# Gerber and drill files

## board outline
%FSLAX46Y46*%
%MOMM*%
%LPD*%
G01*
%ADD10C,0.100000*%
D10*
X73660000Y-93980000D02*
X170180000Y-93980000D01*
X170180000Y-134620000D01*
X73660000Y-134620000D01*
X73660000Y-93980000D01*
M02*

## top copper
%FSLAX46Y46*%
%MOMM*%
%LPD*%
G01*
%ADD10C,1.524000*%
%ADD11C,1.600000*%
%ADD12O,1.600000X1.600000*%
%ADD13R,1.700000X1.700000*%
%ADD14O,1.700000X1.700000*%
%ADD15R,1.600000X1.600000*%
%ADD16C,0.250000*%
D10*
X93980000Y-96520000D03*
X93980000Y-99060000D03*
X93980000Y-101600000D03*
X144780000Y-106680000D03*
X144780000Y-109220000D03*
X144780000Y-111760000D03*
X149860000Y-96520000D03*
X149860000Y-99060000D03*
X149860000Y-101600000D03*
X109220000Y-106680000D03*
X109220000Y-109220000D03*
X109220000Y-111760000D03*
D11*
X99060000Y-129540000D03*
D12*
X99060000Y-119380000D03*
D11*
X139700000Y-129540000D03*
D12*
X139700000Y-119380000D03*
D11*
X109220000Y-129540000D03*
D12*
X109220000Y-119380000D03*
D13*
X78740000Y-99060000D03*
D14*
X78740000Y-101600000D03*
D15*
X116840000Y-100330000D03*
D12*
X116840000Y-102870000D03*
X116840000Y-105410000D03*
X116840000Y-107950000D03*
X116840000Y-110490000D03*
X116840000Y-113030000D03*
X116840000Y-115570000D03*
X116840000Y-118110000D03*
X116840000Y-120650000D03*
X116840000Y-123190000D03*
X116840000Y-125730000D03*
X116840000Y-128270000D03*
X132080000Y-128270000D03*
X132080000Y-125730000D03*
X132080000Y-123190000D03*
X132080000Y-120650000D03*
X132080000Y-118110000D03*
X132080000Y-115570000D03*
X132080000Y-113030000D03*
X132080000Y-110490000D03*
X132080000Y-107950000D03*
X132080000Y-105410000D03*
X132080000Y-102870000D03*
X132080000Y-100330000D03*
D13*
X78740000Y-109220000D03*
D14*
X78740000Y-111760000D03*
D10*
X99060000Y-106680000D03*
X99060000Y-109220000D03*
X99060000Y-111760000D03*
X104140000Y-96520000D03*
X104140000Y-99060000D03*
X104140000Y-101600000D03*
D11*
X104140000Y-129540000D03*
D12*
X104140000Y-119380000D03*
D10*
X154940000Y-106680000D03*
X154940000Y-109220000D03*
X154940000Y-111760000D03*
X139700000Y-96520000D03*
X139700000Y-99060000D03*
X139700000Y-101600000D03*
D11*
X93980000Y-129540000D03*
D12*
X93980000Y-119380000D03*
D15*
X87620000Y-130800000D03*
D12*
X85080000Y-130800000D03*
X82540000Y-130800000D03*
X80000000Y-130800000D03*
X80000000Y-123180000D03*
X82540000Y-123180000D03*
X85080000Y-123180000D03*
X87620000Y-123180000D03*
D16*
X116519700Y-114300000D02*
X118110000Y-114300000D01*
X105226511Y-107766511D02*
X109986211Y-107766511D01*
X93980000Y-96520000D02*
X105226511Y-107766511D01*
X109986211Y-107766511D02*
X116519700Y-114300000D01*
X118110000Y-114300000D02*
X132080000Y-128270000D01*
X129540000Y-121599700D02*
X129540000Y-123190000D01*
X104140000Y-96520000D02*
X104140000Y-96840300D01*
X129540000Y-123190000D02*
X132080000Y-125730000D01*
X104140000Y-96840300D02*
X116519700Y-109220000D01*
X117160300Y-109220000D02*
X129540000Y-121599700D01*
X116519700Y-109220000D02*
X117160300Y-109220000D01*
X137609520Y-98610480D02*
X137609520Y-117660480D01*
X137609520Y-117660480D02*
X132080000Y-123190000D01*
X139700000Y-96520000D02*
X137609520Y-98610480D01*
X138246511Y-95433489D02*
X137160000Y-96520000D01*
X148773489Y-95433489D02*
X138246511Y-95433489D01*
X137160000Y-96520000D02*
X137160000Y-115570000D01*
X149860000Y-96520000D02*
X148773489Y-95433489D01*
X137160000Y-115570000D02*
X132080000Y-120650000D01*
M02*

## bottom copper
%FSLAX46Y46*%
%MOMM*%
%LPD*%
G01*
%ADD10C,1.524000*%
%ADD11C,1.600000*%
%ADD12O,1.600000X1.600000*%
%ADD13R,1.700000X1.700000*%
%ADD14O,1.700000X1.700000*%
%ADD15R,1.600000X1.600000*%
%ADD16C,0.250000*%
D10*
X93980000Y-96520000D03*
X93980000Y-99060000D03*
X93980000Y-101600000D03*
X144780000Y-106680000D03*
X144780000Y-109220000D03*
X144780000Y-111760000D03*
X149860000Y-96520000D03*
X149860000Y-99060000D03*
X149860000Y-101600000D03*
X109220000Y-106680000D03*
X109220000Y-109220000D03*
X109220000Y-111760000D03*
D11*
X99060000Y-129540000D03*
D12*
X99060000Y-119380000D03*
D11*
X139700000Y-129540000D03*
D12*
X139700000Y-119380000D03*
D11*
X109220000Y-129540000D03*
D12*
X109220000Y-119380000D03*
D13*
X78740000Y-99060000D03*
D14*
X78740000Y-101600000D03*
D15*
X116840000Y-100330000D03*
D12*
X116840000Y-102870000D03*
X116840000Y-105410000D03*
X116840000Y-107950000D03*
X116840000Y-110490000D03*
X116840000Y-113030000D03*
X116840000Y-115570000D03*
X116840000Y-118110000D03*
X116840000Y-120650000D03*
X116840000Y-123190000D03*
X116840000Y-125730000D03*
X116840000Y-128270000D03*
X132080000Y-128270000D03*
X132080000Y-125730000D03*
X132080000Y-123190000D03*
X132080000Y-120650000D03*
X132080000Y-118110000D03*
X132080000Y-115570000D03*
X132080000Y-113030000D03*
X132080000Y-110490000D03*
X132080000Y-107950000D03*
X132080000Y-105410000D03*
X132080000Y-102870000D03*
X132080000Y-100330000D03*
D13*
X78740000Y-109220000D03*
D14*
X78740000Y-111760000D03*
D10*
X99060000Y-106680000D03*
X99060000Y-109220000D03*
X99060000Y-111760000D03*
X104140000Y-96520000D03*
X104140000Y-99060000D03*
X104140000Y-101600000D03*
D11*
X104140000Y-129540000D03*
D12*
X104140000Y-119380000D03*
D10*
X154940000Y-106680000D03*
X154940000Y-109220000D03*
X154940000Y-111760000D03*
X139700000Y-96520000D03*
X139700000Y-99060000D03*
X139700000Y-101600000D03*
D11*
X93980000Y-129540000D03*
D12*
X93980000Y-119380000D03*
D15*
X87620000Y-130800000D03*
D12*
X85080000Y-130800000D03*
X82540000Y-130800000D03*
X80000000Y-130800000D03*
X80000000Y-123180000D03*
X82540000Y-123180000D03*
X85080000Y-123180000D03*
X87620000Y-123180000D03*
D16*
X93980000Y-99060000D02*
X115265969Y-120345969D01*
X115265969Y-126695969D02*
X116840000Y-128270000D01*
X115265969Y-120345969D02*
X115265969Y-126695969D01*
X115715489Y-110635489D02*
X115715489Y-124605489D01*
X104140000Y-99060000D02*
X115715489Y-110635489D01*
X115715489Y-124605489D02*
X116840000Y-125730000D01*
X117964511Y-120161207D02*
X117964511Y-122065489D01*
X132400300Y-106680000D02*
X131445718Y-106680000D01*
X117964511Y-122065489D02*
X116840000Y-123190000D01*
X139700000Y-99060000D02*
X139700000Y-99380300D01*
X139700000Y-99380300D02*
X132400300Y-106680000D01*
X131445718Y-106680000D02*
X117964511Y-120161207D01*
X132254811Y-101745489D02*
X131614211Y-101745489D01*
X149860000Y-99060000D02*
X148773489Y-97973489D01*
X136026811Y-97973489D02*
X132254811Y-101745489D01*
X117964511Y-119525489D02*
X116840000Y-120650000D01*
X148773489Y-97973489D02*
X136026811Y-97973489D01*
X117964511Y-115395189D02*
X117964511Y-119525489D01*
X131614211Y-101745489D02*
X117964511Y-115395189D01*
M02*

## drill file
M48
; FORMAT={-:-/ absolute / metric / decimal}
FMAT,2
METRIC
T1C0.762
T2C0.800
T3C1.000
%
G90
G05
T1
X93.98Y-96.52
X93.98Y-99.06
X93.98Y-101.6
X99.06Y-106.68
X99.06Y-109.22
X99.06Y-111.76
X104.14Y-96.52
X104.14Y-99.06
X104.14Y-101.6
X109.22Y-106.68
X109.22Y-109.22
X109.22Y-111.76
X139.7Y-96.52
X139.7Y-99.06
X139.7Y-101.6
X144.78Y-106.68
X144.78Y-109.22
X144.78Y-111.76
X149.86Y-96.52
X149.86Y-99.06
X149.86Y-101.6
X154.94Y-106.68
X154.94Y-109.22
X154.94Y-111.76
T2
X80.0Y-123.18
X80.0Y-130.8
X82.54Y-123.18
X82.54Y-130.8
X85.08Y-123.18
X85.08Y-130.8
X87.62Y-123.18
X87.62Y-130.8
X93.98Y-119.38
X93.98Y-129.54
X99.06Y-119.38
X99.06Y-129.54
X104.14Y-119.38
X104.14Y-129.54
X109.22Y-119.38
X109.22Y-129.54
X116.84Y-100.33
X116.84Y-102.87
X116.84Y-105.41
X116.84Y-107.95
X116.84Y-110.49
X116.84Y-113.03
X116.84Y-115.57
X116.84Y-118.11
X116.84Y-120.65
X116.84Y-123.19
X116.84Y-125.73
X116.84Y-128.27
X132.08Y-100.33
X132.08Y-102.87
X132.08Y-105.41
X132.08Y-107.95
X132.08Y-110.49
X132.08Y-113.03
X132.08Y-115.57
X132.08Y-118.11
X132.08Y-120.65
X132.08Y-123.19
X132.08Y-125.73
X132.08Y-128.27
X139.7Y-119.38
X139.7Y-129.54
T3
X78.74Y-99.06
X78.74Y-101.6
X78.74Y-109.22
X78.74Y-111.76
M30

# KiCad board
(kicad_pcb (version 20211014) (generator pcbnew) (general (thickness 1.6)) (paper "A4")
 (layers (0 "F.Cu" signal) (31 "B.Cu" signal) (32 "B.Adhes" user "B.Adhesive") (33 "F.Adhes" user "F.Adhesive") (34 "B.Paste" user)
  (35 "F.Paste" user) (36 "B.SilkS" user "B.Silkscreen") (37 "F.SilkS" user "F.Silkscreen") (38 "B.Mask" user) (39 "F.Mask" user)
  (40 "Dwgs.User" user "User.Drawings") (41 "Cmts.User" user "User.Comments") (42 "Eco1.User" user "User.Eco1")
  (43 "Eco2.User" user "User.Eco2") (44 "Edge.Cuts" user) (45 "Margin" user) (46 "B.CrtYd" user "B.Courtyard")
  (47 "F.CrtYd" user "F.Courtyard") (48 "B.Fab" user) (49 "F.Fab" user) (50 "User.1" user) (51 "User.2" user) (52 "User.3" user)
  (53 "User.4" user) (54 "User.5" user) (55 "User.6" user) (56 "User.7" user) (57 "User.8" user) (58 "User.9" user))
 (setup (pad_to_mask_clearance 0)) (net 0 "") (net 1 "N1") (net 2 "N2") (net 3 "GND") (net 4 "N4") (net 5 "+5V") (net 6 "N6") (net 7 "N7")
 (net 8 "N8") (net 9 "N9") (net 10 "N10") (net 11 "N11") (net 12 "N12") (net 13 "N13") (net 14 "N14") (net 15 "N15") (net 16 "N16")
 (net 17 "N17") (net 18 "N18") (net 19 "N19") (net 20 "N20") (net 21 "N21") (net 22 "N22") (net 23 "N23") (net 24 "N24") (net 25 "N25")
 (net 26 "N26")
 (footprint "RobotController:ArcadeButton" (layer "F.Cu") (at 93.98 96.52)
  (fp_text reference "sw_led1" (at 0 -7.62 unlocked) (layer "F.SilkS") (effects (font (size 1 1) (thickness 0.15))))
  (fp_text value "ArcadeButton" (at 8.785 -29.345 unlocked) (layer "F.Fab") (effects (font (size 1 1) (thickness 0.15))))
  (pad "1" thru_hole circle (at 0 0) (size 1.524 1.524) (drill 0.762) (layers *.Cu *.Mask) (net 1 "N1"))
  (pad "2" thru_hole circle (at 0 2.54) (size 1.524 1.524) (drill 0.762) (layers *.Cu *.Mask) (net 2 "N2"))
  (pad "3" thru_hole circle (at 0 5.08) (size 1.524 1.524) (drill 0.762) (layers *.Cu *.Mask) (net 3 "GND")))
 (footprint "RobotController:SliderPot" (layer "F.Cu") (at 144.78 106.68)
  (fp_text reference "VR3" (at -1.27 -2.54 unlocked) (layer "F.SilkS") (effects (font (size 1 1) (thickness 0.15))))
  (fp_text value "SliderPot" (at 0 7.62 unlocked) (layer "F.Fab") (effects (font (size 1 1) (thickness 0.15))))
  (pad "1" thru_hole circle (at 0 0) (size 1.524 1.524) (drill 0.762) (layers *.Cu *.Mask) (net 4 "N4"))
  (pad "2" thru_hole circle (at 0 2.54) (size 1.524 1.524) (drill 0.762) (layers *.Cu *.Mask) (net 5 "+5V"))
  (pad "3" thru_hole circle (at 0 5.08) (size 1.524 1.524) (drill 0.762) (layers *.Cu *.Mask) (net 3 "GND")))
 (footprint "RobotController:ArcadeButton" (layer "F.Cu") (at 149.86 96.52)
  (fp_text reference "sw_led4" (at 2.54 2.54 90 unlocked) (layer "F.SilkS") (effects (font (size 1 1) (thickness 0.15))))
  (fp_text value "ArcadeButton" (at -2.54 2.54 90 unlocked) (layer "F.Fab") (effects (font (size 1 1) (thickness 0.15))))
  (pad "1" thru_hole circle (at 0 0) (size 1.524 1.524) (drill 0.762) (layers *.Cu *.Mask) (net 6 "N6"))
  (pad "2" thru_hole circle (at 0 2.54) (size 1.524 1.524) (drill 0.762) (layers *.Cu *.Mask) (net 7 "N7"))
  (pad "3" thru_hole circle (at 0 5.08) (size 1.524 1.524) (drill 0.762) (layers *.Cu *.Mask) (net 3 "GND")))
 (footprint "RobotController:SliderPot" (layer "F.Cu") (at 109.22 106.68)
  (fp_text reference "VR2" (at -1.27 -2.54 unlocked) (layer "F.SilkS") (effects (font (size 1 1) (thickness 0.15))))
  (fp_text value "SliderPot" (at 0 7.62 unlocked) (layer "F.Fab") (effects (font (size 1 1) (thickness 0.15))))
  (pad "1" thru_hole circle (at 0 0) (size 1.524 1.524) (drill 0.762) (layers *.Cu *.Mask) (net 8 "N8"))
  (pad "2" thru_hole circle (at 0 2.54) (size 1.524 1.524) (drill 0.762) (layers *.Cu *.Mask) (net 5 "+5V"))
  (pad "3" thru_hole circle (at 0 5.08) (size 1.524 1.524) (drill 0.762) (layers *.Cu *.Mask) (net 3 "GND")))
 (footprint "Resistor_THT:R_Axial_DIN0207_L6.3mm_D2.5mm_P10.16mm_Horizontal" (layer "F.Cu") (at 99.06 129.54 90)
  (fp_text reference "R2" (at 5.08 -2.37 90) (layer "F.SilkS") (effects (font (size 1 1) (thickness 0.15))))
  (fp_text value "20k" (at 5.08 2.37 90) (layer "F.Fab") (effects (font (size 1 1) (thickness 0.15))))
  (pad "1" thru_hole circle (at 0 0 90) (size 1.6 1.6) (drill 0.8) (layers *.Cu *.Mask) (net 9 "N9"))
  (pad "2" thru_hole oval (at 10.16 0 90) (size 1.6 1.6) (drill 0.8) (layers *.Cu *.Mask) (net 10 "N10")))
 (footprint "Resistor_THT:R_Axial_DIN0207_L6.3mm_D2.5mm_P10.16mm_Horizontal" (layer "F.Cu") (at 139.7 129.54 90)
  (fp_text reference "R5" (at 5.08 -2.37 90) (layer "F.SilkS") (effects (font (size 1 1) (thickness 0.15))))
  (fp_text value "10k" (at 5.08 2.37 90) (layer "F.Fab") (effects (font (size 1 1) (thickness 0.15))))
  (pad "1" thru_hole circle (at 0 0 90) (size 1.6 1.6) (drill 0.8) (layers *.Cu *.Mask) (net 10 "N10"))
  (pad "2" thru_hole oval (at 10.16 0 90) (size 1.6 1.6) (drill 0.8) (layers *.Cu *.Mask) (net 3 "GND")))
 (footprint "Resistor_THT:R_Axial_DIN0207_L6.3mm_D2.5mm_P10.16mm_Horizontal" (layer "F.Cu") (at 109.22 129.54 90)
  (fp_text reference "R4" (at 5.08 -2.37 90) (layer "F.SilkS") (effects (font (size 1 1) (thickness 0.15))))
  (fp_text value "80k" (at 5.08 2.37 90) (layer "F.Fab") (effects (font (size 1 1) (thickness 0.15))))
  (pad "1" thru_hole circle (at 0 0 90) (size 1.6 1.6) (drill 0.8) (layers *.Cu *.Mask) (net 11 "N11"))
  (pad "2" thru_hole oval (at 10.16 0 90) (size 1.6 1.6) (drill 0.8) (layers *.Cu *.Mask) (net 10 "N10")))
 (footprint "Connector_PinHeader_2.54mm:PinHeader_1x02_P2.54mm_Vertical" (layer "F.Cu") (at 78.74 99.06)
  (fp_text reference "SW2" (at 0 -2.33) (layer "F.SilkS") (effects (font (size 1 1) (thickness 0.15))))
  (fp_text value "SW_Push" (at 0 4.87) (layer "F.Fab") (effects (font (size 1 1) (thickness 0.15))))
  (pad "1" thru_hole rect (at 0 0) (size 1.7 1.7) (drill 1) (layers *.Cu *.Mask) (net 3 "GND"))
  (pad "2" thru_hole oval (at 0 2.54) (size 1.7 1.7) (drill 1) (layers *.Cu *.Mask) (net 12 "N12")))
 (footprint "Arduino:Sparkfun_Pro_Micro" (layer "F.Cu") (at 132.08 128.27 180)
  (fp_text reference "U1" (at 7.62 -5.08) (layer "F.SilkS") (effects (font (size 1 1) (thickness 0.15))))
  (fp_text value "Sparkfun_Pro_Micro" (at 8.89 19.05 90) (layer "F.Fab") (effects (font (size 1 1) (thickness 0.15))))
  (pad "1" thru_hole rect locked (at 15.24 27.94 180) (size 1.6 1.6) (drill 0.8) (layers *.Cu *.Mask) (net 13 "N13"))
  (pad "2" thru_hole oval locked (at 15.24 25.4 180) (size 1.6 1.6) (drill 0.8) (layers *.Cu *.Mask) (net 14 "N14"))
  (pad "3" thru_hole oval locked (at 15.24 22.86 180) (size 1.6 1.6) (drill 0.8) (layers *.Cu *.Mask) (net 3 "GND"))
  (pad "4" thru_hole oval locked (at 15.24 20.32 180) (size 1.6 1.6) (drill 0.8) (layers *.Cu *.Mask) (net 3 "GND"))
  (pad "5" thru_hole oval locked (at 15.24 17.78 180) (size 1.6 1.6) (drill 0.8) (layers *.Cu *.Mask) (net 12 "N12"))
  (pad "6" thru_hole oval locked (at 15.24 15.24 180) (size 1.6 1.6) (drill 0.8) (layers *.Cu *.Mask) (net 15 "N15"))
  (pad "7" thru_hole oval locked (at 15.24 12.7 180) (size 1.6 1.6) (drill 0.8) (layers *.Cu *.Mask) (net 10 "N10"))
  (pad "8" thru_hole oval locked (at 15.24 10.16 180) (size 1.6 1.6) (drill 0.8) (layers *.Cu *.Mask) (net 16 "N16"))
  (pad "9" thru_hole oval locked (at 15.24 7.62 180) (size 1.6 1.6) (drill 0.8) (layers *.Cu *.Mask) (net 7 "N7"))
  (pad "10" thru_hole oval locked (at 15.24 5.08 180) (size 1.6 1.6) (drill 0.8) (layers *.Cu *.Mask) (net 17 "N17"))
  (pad "11" thru_hole oval locked (at 15.24 2.54 180) (size 1.6 1.6) (drill 0.8) (layers *.Cu *.Mask) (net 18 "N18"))
  (pad "12" thru_hole oval locked (at 15.24 0 180) (size 1.6 1.6) (drill 0.8) (layers *.Cu *.Mask) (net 2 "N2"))
  (pad "13" thru_hole oval locked (at 0 0 180) (size 1.6 1.6) (drill 0.8) (layers *.Cu *.Mask) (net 1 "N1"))
  (pad "14" thru_hole oval locked (at 0 2.54 180) (size 1.6 1.6) (drill 0.8) (layers *.Cu *.Mask) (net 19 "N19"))
  (pad "15" thru_hole oval locked (at 0 5.08 180) (size 1.6 1.6) (drill 0.8) (layers *.Cu *.Mask) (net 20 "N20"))
  (pad "16" thru_hole oval locked (at 0 7.62 180) (size 1.6 1.6) (drill 0.8) (layers *.Cu *.Mask) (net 6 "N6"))
  (pad "17" thru_hole oval locked (at 0 10.16 180) (size 1.6 1.6) (drill 0.8) (layers *.Cu *.Mask) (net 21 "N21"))
  (pad "18" thru_hole oval locked (at 0 12.7 180) (size 1.6 1.6) (drill 0.8) (layers *.Cu *.Mask) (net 4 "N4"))
  (pad "19" thru_hole oval locked (at 0 15.24 180) (size 1.6 1.6) (drill 0.8) (layers *.Cu *.Mask) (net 8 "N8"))
  (pad "20" thru_hole oval locked (at 0 17.78 180) (size 1.6 1.6) (drill 0.8) (layers *.Cu *.Mask) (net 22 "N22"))
  (pad "21" thru_hole oval locked (at 0 20.32 180) (size 1.6 1.6) (drill 0.8) (layers *.Cu *.Mask) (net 5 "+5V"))
  (pad "22" thru_hole oval locked (at 0 22.86 180) (size 1.6 1.6) (drill 0.8) (layers *.Cu *.Mask) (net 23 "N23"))
  (pad "23" thru_hole oval locked (at 0 25.4 180) (size 1.6 1.6) (drill 0.8) (layers *.Cu *.Mask) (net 3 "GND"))
  (pad "24" thru_hole oval locked (at 0 27.94 180) (size 1.6 1.6) (drill 0.8) (layers *.Cu *.Mask) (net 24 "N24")))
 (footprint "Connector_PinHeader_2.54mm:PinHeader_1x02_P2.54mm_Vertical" (layer "F.Cu") (at 78.74 109.22)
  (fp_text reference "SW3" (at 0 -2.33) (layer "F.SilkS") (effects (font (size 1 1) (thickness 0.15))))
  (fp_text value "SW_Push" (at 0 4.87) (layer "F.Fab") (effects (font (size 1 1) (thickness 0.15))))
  (pad "1" thru_hole rect (at 0 0) (size 1.7 1.7) (drill 1) (layers *.Cu *.Mask) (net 3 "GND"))
  (pad "2" thru_hole oval (at 0 2.54) (size 1.7 1.7) (drill 1) (layers *.Cu *.Mask) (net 15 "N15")))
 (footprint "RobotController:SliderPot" (layer "F.Cu") (at 99.06 106.68)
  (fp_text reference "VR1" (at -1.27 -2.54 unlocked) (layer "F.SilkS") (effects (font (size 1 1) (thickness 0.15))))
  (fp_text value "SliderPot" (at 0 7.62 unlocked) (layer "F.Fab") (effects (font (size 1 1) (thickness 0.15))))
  (pad "1" thru_hole circle (at 0 0) (size 1.524 1.524) (drill 0.762) (layers *.Cu *.Mask) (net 22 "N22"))
  (pad "2" thru_hole circle (at 0 2.54) (size 1.524 1.524) (drill 0.762) (layers *.Cu *.Mask) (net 5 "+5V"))
  (pad "3" thru_hole circle (at 0 5.08) (size 1.524 1.524) (drill 0.762) (layers *.Cu *.Mask) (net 3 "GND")))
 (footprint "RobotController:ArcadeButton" (layer "F.Cu") (at 104.14 96.52)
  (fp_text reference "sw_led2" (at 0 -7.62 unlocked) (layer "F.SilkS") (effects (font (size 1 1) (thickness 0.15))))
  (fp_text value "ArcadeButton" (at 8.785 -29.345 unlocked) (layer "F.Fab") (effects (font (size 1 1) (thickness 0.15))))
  (pad "1" thru_hole circle (at 0 0) (size 1.524 1.524) (drill 0.762) (layers *.Cu *.Mask) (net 19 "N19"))
  (pad "2" thru_hole circle (at 0 2.54) (size 1.524 1.524) (drill 0.762) (layers *.Cu *.Mask) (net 18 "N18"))
  (pad "3" thru_hole circle (at 0 5.08) (size 1.524 1.524) (drill 0.762) (layers *.Cu *.Mask) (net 3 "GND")))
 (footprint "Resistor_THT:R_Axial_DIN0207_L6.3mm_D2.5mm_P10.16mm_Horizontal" (layer "F.Cu") (at 104.14 129.54 90)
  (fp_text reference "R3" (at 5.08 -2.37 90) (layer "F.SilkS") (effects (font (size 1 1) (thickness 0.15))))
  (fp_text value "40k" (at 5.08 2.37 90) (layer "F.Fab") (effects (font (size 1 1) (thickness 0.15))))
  (pad "1" thru_hole circle (at 0 0 90) (size 1.6 1.6) (drill 0.8) (layers *.Cu *.Mask) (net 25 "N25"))
  (pad "2" thru_hole oval (at 10.16 0 90) (size 1.6 1.6) (drill 0.8) (layers *.Cu *.Mask) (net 10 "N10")))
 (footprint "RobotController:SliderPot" (layer "F.Cu") (at 154.94 106.68)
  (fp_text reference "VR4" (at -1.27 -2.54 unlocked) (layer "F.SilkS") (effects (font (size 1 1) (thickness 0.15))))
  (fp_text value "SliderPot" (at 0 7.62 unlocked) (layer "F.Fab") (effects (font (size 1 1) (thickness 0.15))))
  (pad "1" thru_hole circle (at 0 0) (size 1.524 1.524) (drill 0.762) (layers *.Cu *.Mask) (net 21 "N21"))
  (pad "2" thru_hole circle (at 0 2.54) (size 1.524 1.524) (drill 0.762) (layers *.Cu *.Mask) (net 5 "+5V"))
  (pad "3" thru_hole circle (at 0 5.08) (size 1.524 1.524) (drill 0.762) (layers *.Cu *.Mask) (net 3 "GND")))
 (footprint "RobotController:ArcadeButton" (layer "F.Cu") (at 139.7 96.52)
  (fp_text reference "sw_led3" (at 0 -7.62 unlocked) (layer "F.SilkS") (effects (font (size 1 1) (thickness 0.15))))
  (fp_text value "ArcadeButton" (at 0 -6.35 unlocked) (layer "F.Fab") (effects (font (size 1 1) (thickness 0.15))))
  (pad "1" thru_hole circle (at 0 0) (size 1.524 1.524) (drill 0.762) (layers *.Cu *.Mask) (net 20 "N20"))
  (pad "2" thru_hole circle (at 0 2.54) (size 1.524 1.524) (drill 0.762) (layers *.Cu *.Mask) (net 17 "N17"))
  (pad "3" thru_hole circle (at 0 5.08) (size 1.524 1.524) (drill 0.762) (layers *.Cu *.Mask) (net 3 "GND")))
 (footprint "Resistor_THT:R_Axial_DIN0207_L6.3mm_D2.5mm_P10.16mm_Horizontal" (layer "F.Cu") (at 93.98 129.54 90)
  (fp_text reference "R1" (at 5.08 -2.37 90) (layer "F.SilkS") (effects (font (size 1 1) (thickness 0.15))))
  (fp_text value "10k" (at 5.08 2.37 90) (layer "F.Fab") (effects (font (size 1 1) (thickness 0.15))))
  (pad "1" thru_hole circle (at 0 0 90) (size 1.6 1.6) (drill 0.8) (layers *.Cu *.Mask) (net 10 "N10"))
  (pad "2" thru_hole oval (at 10.16 0 90) (size 1.6 1.6) (drill 0.8) (layers *.Cu *.Mask) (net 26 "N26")))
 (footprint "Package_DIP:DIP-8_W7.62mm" (layer "B.Cu") (at 87.62 130.8 90)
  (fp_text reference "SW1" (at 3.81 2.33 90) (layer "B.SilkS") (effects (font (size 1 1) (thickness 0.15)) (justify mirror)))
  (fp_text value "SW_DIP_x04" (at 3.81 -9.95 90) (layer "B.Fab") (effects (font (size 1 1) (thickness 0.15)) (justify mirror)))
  (pad "1" thru_hole rect (at 0 0 90) (size 1.6 1.6) (drill 0.8) (layers *.Cu *.Mask) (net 5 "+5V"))
  (pad "2" thru_hole oval (at 0 -2.54 90) (size 1.6 1.6) (drill 0.8) (layers *.Cu *.Mask) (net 5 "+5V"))
  (pad "3" thru_hole oval (at 0 -5.08 90) (size 1.6 1.6) (drill 0.8) (layers *.Cu *.Mask) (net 5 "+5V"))
  (pad "4" thru_hole oval (at 0 -7.62 90) (size 1.6 1.6) (drill 0.8) (layers *.Cu *.Mask) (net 5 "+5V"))
  (pad "5" thru_hole oval (at 7.62 -7.62 90) (size 1.6 1.6) (drill 0.8) (layers *.Cu *.Mask) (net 11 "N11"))
  (pad "6" thru_hole oval (at 7.62 -5.08 90) (size 1.6 1.6) (drill 0.8) (layers *.Cu *.Mask) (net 25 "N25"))
  (pad "7" thru_hole oval (at 7.62 -2.54 90) (size 1.6 1.6) (drill 0.8) (layers *.Cu *.Mask) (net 9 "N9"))
  (pad "8" thru_hole oval (at 7.62 0 90) (size 1.6 1.6) (drill 0.8) (layers *.Cu *.Mask) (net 26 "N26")))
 (gr_rect (start 73.66 93.98) (end 170.18 134.62) (layer "Edge.Cuts") (width 0.1) (fill none))
 (segment (start 116.5197 114.3) (end 118.11 114.3) (width 0.25) (layer "F.Cu") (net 1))
 (segment (start 105.226511 107.766511) (end 109.986211 107.766511) (width 0.25) (layer "F.Cu") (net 1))
 (segment (start 93.98 96.52) (end 105.226511 107.766511) (width 0.25) (layer "F.Cu") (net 1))
 (segment (start 109.986211 107.766511) (end 116.5197 114.3) (width 0.25) (layer "F.Cu") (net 1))
 (segment (start 118.11 114.3) (end 132.08 128.27) (width 0.25) (layer "F.Cu") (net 1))
 (segment (start 93.98 99.06) (end 115.265969 120.345969) (width 0.25) (layer "B.Cu") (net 2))
 (segment (start 115.265969 126.695969) (end 116.84 128.27) (width 0.25) (layer "B.Cu") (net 2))
 (segment (start 115.265969 120.345969) (end 115.265969 126.695969) (width 0.25) (layer "B.Cu") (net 2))
 (segment (start 129.54 121.5997) (end 129.54 123.19) (width 0.25) (layer "F.Cu") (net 19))
 (segment (start 104.14 96.52) (end 104.14 96.8403) (width 0.25) (layer "F.Cu") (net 19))
 (segment (start 129.54 123.19) (end 132.08 125.73) (width 0.25) (layer "F.Cu") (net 19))
 (segment (start 104.14 96.8403) (end 116.5197 109.22) (width 0.25) (layer "F.Cu") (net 19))
 (segment (start 117.1603 109.22) (end 129.54 121.5997) (width 0.25) (layer "F.Cu") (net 19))
 (segment (start 116.5197 109.22) (end 117.1603 109.22) (width 0.25) (layer "F.Cu") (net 19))
 (segment (start 115.715489 110.635489) (end 115.715489 124.605489) (width 0.25) (layer "B.Cu") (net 18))
 (segment (start 104.14 99.06) (end 115.715489 110.635489) (width 0.25) (layer "B.Cu") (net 18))
 (segment (start 115.715489 124.605489) (end 116.84 125.73) (width 0.25) (layer "B.Cu") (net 18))
 (segment (start 137.60952 98.61048) (end 137.60952 117.66048) (width 0.25) (layer "F.Cu") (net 20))
 (segment (start 137.60952 117.66048) (end 132.08 123.19) (width 0.25) (layer "F.Cu") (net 20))
 (segment (start 139.7 96.52) (end 137.60952 98.61048) (width 0.25) (layer "F.Cu") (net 20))
 (segment (start 117.964511 120.161207) (end 117.964511 122.065489) (width 0.25) (layer "B.Cu") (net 17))
 (segment (start 132.4003 106.68) (end 131.445718 106.68) (width 0.25) (layer "B.Cu") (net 17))
 (segment (start 117.964511 122.065489) (end 116.84 123.19) (width 0.25) (layer "B.Cu") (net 17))
 (segment (start 139.7 99.06) (end 139.7 99.3803) (width 0.25) (layer "B.Cu") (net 17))
 (segment (start 139.7 99.3803) (end 132.4003 106.68) (width 0.25) (layer "B.Cu") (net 17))
 (segment (start 131.445718 106.68) (end 117.964511 120.161207) (width 0.25) (layer "B.Cu") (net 17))
 (segment (start 138.246511 95.433489) (end 137.16 96.52) (width 0.25) (layer "F.Cu") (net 6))
 (segment (start 148.773489 95.433489) (end 138.246511 95.433489) (width 0.25) (layer "F.Cu") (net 6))
 (segment (start 137.16 96.52) (end 137.16 115.57) (width 0.25) (layer "F.Cu") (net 6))
 (segment (start 149.86 96.52) (end 148.773489 95.433489) (width 0.25) (layer "F.Cu") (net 6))
 (segment (start 137.16 115.57) (end 132.08 120.65) (width 0.25) (layer "F.Cu") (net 6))
 (segment (start 132.254811 101.745489) (end 131.614211 101.745489) (width 0.25) (layer "B.Cu") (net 7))
 (segment (start 149.86 99.06) (end 148.773489 97.973489) (width 0.25) (layer "B.Cu") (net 7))
 (segment (start 136.026811 97.973489) (end 132.254811 101.745489) (width 0.25) (layer "B.Cu") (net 7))
 (segment (start 117.964511 119.525489) (end 116.84 120.65) (width 0.25) (layer "B.Cu") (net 7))
 (segment (start 148.773489 97.973489) (end 136.026811 97.973489) (width 0.25) (layer "B.Cu") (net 7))
 (segment (start 117.964511 115.395189) (end 117.964511 119.525489) (width 0.25) (layer "B.Cu") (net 7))
 (segment (start 131.614211 101.745489) (end 117.964511 115.395189) (width 0.25) (layer "B.Cu") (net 7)))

